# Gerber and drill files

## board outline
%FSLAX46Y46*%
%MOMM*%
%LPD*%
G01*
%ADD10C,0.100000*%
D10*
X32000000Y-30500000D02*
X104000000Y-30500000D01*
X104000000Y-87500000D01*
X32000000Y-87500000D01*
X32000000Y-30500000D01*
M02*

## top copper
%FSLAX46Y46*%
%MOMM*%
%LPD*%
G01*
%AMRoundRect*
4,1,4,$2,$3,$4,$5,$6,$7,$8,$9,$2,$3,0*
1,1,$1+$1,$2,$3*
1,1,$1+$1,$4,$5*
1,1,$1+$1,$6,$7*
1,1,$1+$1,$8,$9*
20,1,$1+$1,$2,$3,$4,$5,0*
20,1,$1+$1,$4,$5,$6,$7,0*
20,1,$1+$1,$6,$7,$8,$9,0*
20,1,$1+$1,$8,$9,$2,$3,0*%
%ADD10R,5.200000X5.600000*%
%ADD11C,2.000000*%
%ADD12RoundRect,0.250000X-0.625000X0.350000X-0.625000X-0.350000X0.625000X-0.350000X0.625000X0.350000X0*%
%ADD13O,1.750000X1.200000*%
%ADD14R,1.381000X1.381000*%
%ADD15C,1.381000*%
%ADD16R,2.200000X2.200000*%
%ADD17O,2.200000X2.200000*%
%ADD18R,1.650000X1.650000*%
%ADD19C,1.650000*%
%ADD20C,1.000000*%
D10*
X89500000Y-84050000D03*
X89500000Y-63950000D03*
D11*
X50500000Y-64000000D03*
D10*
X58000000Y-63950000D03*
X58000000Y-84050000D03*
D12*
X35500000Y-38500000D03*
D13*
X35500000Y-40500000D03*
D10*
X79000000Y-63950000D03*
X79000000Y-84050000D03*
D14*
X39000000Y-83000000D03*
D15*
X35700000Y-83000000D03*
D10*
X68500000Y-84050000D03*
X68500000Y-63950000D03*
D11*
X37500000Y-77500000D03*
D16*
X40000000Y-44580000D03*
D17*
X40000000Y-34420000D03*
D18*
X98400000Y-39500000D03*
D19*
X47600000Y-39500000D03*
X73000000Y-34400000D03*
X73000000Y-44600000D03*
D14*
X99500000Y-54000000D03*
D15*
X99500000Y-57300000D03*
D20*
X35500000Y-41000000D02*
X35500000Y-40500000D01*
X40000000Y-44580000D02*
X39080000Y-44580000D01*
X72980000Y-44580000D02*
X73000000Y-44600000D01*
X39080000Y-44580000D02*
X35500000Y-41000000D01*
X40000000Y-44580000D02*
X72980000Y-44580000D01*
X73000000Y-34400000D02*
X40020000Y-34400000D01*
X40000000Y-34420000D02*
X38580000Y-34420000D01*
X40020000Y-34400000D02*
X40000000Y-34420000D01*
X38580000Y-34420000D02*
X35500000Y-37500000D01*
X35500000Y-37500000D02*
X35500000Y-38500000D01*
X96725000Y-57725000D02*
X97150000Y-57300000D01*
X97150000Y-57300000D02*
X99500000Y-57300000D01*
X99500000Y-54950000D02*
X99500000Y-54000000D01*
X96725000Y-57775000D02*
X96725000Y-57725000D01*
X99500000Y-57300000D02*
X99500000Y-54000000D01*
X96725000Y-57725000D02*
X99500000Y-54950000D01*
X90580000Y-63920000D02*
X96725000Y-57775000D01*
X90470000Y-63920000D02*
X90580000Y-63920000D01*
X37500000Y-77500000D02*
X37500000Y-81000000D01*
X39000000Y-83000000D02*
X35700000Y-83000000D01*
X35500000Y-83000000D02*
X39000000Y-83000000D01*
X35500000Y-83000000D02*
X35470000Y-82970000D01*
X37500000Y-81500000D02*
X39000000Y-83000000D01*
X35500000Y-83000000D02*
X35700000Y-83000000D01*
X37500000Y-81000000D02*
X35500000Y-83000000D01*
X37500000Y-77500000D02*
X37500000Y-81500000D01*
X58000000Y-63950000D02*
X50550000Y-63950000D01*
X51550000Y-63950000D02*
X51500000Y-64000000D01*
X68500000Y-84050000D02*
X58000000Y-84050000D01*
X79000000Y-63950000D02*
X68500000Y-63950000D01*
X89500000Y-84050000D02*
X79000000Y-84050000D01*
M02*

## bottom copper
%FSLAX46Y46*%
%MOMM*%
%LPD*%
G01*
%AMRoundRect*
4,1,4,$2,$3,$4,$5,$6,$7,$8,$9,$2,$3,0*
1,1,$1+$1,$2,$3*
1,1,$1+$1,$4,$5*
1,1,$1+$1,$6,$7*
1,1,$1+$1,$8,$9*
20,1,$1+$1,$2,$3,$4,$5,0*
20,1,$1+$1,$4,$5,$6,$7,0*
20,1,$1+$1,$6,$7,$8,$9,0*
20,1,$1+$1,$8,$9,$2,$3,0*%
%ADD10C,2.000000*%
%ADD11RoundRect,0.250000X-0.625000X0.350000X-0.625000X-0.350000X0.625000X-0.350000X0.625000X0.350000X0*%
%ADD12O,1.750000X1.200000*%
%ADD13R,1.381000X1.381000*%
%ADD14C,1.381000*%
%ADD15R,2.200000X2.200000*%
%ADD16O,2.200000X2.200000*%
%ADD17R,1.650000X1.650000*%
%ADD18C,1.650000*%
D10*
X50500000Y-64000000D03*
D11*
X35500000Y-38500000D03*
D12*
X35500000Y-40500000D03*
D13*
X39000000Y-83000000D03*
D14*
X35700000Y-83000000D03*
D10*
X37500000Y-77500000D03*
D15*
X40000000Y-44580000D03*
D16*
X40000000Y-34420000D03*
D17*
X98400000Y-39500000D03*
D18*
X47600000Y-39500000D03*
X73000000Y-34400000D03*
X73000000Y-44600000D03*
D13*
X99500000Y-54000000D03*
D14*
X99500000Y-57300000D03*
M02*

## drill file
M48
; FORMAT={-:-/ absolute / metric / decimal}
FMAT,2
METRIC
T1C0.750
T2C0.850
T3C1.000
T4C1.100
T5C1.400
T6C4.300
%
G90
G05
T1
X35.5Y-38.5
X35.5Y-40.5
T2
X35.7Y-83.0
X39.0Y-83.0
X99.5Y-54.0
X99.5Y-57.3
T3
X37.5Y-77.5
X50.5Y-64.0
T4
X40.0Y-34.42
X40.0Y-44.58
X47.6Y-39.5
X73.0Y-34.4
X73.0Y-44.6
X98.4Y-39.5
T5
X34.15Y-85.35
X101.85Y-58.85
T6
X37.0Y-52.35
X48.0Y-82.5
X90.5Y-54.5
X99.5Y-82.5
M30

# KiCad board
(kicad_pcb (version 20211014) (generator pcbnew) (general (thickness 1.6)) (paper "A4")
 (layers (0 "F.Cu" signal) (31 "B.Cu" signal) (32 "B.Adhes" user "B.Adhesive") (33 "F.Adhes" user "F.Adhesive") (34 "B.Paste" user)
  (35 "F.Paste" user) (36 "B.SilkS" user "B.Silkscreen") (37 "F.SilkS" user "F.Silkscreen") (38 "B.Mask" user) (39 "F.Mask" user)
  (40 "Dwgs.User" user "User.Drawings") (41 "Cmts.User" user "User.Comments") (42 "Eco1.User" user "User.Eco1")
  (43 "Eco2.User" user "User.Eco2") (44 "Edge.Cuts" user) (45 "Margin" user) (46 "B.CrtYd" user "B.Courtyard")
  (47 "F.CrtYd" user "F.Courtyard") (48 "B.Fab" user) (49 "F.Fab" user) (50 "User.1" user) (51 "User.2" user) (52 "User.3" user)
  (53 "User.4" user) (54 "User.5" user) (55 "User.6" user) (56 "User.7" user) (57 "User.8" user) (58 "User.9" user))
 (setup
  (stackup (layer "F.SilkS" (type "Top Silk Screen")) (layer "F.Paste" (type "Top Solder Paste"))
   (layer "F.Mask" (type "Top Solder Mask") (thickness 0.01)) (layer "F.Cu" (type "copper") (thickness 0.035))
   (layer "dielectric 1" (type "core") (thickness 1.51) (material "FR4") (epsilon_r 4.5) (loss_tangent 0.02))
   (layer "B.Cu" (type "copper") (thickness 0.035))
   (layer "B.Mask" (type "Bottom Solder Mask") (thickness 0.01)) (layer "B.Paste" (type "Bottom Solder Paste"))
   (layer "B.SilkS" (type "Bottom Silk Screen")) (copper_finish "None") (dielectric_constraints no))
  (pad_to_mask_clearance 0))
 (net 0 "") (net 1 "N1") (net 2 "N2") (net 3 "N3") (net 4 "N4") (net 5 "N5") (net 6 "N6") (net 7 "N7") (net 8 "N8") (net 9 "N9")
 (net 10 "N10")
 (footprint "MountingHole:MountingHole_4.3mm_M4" (layer "F.Cu") (at 90.5 54.5)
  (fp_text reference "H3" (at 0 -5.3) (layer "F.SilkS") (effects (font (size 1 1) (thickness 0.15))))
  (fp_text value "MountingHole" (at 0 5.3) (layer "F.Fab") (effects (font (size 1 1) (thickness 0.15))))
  (pad "" np_thru_hole circle (at 0 0) (size 4.3 4.3) (drill 4.3) (layers *.Cu *.Mask)))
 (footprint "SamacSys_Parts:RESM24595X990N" (layer "F.Cu") (at 89.5 74 90)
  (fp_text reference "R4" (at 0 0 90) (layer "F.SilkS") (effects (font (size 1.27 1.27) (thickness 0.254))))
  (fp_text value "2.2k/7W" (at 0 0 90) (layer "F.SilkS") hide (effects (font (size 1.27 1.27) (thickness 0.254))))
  (pad "1" smd rect locked (at -10.05 0 180) (size 5.2 5.6) (layers "F.Cu" "F.Paste" "F.Mask") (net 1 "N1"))
  (pad "2" smd rect locked (at 10.05 0 180) (size 5.2 5.6) (layers "F.Cu" "F.Paste" "F.Mask") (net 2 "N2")))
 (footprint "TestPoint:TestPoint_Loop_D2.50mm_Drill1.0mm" (layer "F.Cu") (at 50.5 64)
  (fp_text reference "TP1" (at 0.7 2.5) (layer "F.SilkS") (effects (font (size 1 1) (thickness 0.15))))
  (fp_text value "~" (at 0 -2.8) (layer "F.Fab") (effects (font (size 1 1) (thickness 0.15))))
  (pad "1" thru_hole circle (at 0 0) (size 2 2) (drill 1) (layers *.Cu *.Mask) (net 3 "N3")))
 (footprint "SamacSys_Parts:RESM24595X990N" (layer "F.Cu") (at 58 74 -90)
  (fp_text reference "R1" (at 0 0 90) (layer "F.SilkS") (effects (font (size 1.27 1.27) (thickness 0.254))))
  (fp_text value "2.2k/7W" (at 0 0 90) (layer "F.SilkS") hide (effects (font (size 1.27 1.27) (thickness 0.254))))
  (pad "1" smd rect locked (at -10.05 0) (size 5.2 5.6) (layers "F.Cu" "F.Paste" "F.Mask") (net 3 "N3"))
  (pad "2" smd rect locked (at 10.05 0) (size 5.2 5.6) (layers "F.Cu" "F.Paste" "F.Mask") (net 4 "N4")))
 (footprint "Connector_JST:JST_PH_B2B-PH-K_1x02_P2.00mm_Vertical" (layer "F.Cu") (at 35.5 38.5 -90)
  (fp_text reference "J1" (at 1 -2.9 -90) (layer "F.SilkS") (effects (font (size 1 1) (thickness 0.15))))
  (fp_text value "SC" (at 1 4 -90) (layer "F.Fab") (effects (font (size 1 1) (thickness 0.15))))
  (pad "1" thru_hole roundrect (at 0 0 270) (size 1.2 1.75) (drill 0.75) (layers *.Cu *.Mask) (roundrect_rratio 0.208333) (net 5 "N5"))
  (pad "2" thru_hole oval (at 2 0 270) (size 1.2 1.75) (drill 0.75) (layers *.Cu *.Mask) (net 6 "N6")))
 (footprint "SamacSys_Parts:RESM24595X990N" (layer "F.Cu") (at 79 74 -90)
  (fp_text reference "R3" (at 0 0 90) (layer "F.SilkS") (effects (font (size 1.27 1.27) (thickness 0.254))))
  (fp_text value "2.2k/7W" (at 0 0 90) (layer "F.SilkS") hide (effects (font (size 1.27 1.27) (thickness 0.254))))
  (pad "1" smd rect locked (at -10.05 0) (size 5.2 5.6) (layers "F.Cu" "F.Paste" "F.Mask") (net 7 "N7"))
  (pad "2" smd rect locked (at 10.05 0) (size 5.2 5.6) (layers "F.Cu" "F.Paste" "F.Mask") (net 1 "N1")))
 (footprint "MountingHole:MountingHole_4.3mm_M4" (layer "F.Cu") (at 37 52.35)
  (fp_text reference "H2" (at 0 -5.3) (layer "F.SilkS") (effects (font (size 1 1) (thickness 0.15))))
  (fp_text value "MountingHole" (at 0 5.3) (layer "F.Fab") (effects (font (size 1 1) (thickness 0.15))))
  (pad "" np_thru_hole circle (at 0 0) (size 4.3 4.3) (drill 4.3) (layers *.Cu *.Mask)))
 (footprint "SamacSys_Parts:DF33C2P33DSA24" (layer "F.Cu") (at 39 83 180)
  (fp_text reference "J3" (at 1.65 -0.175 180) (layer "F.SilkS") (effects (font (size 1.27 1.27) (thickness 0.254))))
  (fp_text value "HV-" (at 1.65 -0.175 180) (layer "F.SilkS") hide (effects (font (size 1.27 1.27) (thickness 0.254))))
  (pad "" np_thru_hole circle locked (at 4.85 -2.35 180) (size 1.4 1.4) (drill 1.4) (layers *.Cu *.Mask))
  (pad "1" thru_hole rect locked (at 0 0 180) (size 1.381 1.381) (drill 0.85) (layers *.Cu *.Mask) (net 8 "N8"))
  (pad "2" thru_hole circle locked (at 3.3 0 180) (size 1.381 1.381) (drill 0.85) (layers *.Cu *.Mask) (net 8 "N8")))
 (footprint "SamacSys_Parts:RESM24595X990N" (layer "F.Cu") (at 68.5 74 90)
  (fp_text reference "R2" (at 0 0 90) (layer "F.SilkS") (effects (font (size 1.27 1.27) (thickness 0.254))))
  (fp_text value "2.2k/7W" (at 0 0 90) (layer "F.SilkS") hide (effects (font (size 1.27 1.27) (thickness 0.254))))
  (pad "1" smd rect locked (at -10.05 0 180) (size 5.2 5.6) (layers "F.Cu" "F.Paste" "F.Mask") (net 4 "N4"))
  (pad "2" smd rect locked (at 10.05 0 180) (size 5.2 5.6) (layers "F.Cu" "F.Paste" "F.Mask") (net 7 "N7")))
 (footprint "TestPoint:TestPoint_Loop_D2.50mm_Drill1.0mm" (layer "F.Cu") (at 37.5 77.5 -90)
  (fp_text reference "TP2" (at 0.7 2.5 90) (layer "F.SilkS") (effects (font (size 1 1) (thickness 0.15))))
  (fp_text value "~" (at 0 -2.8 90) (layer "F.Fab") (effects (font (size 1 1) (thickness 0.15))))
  (pad "1" thru_hole circle (at 0 0 270) (size 2 2) (drill 1) (layers *.Cu *.Mask) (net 8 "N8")))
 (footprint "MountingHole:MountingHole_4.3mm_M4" (layer "F.Cu") (at 99.5 82.5)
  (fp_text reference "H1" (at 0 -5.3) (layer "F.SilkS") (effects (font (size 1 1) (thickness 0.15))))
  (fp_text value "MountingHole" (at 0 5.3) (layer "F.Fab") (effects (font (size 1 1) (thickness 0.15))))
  (pad "" np_thru_hole circle (at 0 0) (size 4.3 4.3) (drill 4.3) (layers *.Cu *.Mask)))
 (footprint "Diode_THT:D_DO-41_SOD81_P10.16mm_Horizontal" (layer "F.Cu") (at 40 44.58 90)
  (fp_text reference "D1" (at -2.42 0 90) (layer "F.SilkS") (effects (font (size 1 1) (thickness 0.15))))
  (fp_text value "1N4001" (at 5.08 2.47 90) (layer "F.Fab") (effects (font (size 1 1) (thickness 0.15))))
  (pad "1" thru_hole rect (at 0 0 90) (size 2.2 2.2) (drill 1.1) (layers *.Cu *.Mask) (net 6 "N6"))
  (pad "2" thru_hole oval (at 10.16 0 90) (size 2.2 2.2) (drill 1.1) (layers *.Cu *.Mask) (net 5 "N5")))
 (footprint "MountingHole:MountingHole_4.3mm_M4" (layer "F.Cu") (at 48 82.5)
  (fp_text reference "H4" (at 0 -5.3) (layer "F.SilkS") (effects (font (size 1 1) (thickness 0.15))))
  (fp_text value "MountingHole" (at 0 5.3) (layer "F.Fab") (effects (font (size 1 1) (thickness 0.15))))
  (pad "" np_thru_hole circle (at 0 0) (size 4.3 4.3) (drill 4.3) (layers *.Cu *.Mask)))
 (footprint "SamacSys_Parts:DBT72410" (layer "F.Cu") (at 98.4 39.5 180)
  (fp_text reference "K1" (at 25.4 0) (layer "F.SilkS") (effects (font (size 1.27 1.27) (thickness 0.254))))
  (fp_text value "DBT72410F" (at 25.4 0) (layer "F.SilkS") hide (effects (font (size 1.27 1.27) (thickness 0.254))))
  (pad "1" thru_hole rect (at 0 0 180) (size 1.65 1.65) (drill 1.1) (layers *.Cu *.Mask) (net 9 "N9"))
  (pad "2" thru_hole circle (at 50.8 0 180) (size 1.65 1.65) (drill 1.1) (layers *.Cu *.Mask) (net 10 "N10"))
  (pad "3" thru_hole circle (at 25.4 5.1 180) (size 1.65 1.65) (drill 1.1) (layers *.Cu *.Mask) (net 5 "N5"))
  (pad "4" thru_hole circle (at 25.4 -5.1 180) (size 1.65 1.65) (drill 1.1) (layers *.Cu *.Mask) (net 6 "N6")))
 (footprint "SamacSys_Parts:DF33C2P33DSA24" (layer "F.Cu") (at 99.5 54 -90)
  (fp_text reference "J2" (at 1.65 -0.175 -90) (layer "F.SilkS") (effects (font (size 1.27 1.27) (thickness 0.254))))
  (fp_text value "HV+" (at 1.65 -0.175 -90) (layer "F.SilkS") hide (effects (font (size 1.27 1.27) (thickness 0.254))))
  (pad "" np_thru_hole circle locked (at 4.85 -2.35 270) (size 1.4 1.4) (drill 1.4) (layers *.Cu *.Mask))
  (pad "1" thru_hole rect locked (at 0 0 270) (size 1.381 1.381) (drill 0.85) (layers *.Cu *.Mask) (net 2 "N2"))
  (pad "2" thru_hole circle locked (at 3.3 0 270) (size 1.381 1.381) (drill 0.85) (layers *.Cu *.Mask) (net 2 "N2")))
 (gr_rect (start 104 30.5) (end 32 87.5) (layer "Edge.Cuts") (width 0.1) (fill none))
 (segment (start 35.5 41) (end 35.5 40.5) (width 1) (layer "F.Cu") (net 6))
 (segment (start 40 44.58) (end 39.08 44.58) (width 1) (layer "F.Cu") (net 6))
 (segment (start 72.98 44.58) (end 73 44.6) (width 1) (layer "F.Cu") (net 6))
 (segment (start 39.08 44.58) (end 35.5 41) (width 1) (layer "F.Cu") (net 6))
 (segment (start 40 44.58) (end 72.98 44.58) (width 1) (layer "F.Cu") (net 6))
 (segment (start 73 34.4) (end 40.02 34.4) (width 1) (layer "F.Cu") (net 5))
 (segment (start 40 34.42) (end 38.58 34.42) (width 1) (layer "F.Cu") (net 5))
 (segment (start 40.02 34.4) (end 40 34.42) (width 1) (layer "F.Cu") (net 5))
 (segment (start 38.58 34.42) (end 35.5 37.5) (width 1) (layer "F.Cu") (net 5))
 (segment (start 35.5 37.5) (end 35.5 38.5) (width 1) (layer "F.Cu") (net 5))
 (segment (start 96.725 57.725) (end 97.15 57.3) (width 1) (layer "F.Cu") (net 2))
 (segment (start 97.15 57.3) (end 99.5 57.3) (width 1) (layer "F.Cu") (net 2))
 (segment (start 99.5 54.95) (end 99.5 54) (width 1) (layer "F.Cu") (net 2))
 (segment (start 96.725 57.775) (end 96.725 57.725) (width 1) (layer "F.Cu") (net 2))
 (segment (start 99.5 57.3) (end 99.5 54) (width 1) (layer "F.Cu") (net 2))
 (segment (start 96.725 57.725) (end 99.5 54.95) (width 1) (layer "F.Cu") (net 2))
 (segment (start 90.58 63.92) (end 96.725 57.775) (width 1) (layer "F.Cu") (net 2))
 (segment (start 90.47 63.92) (end 90.58 63.92) (width 1) (layer "F.Cu") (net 2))
 (segment (start 37.5 77.5) (end 37.5 81) (width 1) (layer "F.Cu") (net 8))
 (segment (start 39 83) (end 35.7 83) (width 1) (layer "F.Cu") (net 8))
 (segment (start 35.5 83) (end 39 83) (width 1) (layer "F.Cu") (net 8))
 (segment (start 35.5 83) (end 35.47 82.97) (width 1) (layer "F.Cu") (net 8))
 (segment (start 37.5 81.5) (end 39 83) (width 1) (layer "F.Cu") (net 8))
 (segment (start 35.5 83) (end 35.7 83) (width 1) (layer "F.Cu") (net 8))
 (segment (start 37.5 81) (end 35.5 83) (width 1) (layer "F.Cu") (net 8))
 (segment (start 37.5 77.5) (end 37.5 81.5) (width 1) (layer "F.Cu") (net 8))
 (segment (start 58 63.95) (end 50.55 63.95) (width 1) (layer "F.Cu") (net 3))
 (segment (start 51.55 63.95) (end 51.5 64) (width 1) (layer "F.Cu") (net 3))
 (segment (start 68.5 84.05) (end 58 84.05) (width 1) (layer "F.Cu") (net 4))
 (segment (start 79 63.95) (end 68.5 63.95) (width 1) (layer "F.Cu") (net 7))
 (segment (start 89.5 84.05) (end 79 84.05) (width 1) (layer "F.Cu") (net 1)))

